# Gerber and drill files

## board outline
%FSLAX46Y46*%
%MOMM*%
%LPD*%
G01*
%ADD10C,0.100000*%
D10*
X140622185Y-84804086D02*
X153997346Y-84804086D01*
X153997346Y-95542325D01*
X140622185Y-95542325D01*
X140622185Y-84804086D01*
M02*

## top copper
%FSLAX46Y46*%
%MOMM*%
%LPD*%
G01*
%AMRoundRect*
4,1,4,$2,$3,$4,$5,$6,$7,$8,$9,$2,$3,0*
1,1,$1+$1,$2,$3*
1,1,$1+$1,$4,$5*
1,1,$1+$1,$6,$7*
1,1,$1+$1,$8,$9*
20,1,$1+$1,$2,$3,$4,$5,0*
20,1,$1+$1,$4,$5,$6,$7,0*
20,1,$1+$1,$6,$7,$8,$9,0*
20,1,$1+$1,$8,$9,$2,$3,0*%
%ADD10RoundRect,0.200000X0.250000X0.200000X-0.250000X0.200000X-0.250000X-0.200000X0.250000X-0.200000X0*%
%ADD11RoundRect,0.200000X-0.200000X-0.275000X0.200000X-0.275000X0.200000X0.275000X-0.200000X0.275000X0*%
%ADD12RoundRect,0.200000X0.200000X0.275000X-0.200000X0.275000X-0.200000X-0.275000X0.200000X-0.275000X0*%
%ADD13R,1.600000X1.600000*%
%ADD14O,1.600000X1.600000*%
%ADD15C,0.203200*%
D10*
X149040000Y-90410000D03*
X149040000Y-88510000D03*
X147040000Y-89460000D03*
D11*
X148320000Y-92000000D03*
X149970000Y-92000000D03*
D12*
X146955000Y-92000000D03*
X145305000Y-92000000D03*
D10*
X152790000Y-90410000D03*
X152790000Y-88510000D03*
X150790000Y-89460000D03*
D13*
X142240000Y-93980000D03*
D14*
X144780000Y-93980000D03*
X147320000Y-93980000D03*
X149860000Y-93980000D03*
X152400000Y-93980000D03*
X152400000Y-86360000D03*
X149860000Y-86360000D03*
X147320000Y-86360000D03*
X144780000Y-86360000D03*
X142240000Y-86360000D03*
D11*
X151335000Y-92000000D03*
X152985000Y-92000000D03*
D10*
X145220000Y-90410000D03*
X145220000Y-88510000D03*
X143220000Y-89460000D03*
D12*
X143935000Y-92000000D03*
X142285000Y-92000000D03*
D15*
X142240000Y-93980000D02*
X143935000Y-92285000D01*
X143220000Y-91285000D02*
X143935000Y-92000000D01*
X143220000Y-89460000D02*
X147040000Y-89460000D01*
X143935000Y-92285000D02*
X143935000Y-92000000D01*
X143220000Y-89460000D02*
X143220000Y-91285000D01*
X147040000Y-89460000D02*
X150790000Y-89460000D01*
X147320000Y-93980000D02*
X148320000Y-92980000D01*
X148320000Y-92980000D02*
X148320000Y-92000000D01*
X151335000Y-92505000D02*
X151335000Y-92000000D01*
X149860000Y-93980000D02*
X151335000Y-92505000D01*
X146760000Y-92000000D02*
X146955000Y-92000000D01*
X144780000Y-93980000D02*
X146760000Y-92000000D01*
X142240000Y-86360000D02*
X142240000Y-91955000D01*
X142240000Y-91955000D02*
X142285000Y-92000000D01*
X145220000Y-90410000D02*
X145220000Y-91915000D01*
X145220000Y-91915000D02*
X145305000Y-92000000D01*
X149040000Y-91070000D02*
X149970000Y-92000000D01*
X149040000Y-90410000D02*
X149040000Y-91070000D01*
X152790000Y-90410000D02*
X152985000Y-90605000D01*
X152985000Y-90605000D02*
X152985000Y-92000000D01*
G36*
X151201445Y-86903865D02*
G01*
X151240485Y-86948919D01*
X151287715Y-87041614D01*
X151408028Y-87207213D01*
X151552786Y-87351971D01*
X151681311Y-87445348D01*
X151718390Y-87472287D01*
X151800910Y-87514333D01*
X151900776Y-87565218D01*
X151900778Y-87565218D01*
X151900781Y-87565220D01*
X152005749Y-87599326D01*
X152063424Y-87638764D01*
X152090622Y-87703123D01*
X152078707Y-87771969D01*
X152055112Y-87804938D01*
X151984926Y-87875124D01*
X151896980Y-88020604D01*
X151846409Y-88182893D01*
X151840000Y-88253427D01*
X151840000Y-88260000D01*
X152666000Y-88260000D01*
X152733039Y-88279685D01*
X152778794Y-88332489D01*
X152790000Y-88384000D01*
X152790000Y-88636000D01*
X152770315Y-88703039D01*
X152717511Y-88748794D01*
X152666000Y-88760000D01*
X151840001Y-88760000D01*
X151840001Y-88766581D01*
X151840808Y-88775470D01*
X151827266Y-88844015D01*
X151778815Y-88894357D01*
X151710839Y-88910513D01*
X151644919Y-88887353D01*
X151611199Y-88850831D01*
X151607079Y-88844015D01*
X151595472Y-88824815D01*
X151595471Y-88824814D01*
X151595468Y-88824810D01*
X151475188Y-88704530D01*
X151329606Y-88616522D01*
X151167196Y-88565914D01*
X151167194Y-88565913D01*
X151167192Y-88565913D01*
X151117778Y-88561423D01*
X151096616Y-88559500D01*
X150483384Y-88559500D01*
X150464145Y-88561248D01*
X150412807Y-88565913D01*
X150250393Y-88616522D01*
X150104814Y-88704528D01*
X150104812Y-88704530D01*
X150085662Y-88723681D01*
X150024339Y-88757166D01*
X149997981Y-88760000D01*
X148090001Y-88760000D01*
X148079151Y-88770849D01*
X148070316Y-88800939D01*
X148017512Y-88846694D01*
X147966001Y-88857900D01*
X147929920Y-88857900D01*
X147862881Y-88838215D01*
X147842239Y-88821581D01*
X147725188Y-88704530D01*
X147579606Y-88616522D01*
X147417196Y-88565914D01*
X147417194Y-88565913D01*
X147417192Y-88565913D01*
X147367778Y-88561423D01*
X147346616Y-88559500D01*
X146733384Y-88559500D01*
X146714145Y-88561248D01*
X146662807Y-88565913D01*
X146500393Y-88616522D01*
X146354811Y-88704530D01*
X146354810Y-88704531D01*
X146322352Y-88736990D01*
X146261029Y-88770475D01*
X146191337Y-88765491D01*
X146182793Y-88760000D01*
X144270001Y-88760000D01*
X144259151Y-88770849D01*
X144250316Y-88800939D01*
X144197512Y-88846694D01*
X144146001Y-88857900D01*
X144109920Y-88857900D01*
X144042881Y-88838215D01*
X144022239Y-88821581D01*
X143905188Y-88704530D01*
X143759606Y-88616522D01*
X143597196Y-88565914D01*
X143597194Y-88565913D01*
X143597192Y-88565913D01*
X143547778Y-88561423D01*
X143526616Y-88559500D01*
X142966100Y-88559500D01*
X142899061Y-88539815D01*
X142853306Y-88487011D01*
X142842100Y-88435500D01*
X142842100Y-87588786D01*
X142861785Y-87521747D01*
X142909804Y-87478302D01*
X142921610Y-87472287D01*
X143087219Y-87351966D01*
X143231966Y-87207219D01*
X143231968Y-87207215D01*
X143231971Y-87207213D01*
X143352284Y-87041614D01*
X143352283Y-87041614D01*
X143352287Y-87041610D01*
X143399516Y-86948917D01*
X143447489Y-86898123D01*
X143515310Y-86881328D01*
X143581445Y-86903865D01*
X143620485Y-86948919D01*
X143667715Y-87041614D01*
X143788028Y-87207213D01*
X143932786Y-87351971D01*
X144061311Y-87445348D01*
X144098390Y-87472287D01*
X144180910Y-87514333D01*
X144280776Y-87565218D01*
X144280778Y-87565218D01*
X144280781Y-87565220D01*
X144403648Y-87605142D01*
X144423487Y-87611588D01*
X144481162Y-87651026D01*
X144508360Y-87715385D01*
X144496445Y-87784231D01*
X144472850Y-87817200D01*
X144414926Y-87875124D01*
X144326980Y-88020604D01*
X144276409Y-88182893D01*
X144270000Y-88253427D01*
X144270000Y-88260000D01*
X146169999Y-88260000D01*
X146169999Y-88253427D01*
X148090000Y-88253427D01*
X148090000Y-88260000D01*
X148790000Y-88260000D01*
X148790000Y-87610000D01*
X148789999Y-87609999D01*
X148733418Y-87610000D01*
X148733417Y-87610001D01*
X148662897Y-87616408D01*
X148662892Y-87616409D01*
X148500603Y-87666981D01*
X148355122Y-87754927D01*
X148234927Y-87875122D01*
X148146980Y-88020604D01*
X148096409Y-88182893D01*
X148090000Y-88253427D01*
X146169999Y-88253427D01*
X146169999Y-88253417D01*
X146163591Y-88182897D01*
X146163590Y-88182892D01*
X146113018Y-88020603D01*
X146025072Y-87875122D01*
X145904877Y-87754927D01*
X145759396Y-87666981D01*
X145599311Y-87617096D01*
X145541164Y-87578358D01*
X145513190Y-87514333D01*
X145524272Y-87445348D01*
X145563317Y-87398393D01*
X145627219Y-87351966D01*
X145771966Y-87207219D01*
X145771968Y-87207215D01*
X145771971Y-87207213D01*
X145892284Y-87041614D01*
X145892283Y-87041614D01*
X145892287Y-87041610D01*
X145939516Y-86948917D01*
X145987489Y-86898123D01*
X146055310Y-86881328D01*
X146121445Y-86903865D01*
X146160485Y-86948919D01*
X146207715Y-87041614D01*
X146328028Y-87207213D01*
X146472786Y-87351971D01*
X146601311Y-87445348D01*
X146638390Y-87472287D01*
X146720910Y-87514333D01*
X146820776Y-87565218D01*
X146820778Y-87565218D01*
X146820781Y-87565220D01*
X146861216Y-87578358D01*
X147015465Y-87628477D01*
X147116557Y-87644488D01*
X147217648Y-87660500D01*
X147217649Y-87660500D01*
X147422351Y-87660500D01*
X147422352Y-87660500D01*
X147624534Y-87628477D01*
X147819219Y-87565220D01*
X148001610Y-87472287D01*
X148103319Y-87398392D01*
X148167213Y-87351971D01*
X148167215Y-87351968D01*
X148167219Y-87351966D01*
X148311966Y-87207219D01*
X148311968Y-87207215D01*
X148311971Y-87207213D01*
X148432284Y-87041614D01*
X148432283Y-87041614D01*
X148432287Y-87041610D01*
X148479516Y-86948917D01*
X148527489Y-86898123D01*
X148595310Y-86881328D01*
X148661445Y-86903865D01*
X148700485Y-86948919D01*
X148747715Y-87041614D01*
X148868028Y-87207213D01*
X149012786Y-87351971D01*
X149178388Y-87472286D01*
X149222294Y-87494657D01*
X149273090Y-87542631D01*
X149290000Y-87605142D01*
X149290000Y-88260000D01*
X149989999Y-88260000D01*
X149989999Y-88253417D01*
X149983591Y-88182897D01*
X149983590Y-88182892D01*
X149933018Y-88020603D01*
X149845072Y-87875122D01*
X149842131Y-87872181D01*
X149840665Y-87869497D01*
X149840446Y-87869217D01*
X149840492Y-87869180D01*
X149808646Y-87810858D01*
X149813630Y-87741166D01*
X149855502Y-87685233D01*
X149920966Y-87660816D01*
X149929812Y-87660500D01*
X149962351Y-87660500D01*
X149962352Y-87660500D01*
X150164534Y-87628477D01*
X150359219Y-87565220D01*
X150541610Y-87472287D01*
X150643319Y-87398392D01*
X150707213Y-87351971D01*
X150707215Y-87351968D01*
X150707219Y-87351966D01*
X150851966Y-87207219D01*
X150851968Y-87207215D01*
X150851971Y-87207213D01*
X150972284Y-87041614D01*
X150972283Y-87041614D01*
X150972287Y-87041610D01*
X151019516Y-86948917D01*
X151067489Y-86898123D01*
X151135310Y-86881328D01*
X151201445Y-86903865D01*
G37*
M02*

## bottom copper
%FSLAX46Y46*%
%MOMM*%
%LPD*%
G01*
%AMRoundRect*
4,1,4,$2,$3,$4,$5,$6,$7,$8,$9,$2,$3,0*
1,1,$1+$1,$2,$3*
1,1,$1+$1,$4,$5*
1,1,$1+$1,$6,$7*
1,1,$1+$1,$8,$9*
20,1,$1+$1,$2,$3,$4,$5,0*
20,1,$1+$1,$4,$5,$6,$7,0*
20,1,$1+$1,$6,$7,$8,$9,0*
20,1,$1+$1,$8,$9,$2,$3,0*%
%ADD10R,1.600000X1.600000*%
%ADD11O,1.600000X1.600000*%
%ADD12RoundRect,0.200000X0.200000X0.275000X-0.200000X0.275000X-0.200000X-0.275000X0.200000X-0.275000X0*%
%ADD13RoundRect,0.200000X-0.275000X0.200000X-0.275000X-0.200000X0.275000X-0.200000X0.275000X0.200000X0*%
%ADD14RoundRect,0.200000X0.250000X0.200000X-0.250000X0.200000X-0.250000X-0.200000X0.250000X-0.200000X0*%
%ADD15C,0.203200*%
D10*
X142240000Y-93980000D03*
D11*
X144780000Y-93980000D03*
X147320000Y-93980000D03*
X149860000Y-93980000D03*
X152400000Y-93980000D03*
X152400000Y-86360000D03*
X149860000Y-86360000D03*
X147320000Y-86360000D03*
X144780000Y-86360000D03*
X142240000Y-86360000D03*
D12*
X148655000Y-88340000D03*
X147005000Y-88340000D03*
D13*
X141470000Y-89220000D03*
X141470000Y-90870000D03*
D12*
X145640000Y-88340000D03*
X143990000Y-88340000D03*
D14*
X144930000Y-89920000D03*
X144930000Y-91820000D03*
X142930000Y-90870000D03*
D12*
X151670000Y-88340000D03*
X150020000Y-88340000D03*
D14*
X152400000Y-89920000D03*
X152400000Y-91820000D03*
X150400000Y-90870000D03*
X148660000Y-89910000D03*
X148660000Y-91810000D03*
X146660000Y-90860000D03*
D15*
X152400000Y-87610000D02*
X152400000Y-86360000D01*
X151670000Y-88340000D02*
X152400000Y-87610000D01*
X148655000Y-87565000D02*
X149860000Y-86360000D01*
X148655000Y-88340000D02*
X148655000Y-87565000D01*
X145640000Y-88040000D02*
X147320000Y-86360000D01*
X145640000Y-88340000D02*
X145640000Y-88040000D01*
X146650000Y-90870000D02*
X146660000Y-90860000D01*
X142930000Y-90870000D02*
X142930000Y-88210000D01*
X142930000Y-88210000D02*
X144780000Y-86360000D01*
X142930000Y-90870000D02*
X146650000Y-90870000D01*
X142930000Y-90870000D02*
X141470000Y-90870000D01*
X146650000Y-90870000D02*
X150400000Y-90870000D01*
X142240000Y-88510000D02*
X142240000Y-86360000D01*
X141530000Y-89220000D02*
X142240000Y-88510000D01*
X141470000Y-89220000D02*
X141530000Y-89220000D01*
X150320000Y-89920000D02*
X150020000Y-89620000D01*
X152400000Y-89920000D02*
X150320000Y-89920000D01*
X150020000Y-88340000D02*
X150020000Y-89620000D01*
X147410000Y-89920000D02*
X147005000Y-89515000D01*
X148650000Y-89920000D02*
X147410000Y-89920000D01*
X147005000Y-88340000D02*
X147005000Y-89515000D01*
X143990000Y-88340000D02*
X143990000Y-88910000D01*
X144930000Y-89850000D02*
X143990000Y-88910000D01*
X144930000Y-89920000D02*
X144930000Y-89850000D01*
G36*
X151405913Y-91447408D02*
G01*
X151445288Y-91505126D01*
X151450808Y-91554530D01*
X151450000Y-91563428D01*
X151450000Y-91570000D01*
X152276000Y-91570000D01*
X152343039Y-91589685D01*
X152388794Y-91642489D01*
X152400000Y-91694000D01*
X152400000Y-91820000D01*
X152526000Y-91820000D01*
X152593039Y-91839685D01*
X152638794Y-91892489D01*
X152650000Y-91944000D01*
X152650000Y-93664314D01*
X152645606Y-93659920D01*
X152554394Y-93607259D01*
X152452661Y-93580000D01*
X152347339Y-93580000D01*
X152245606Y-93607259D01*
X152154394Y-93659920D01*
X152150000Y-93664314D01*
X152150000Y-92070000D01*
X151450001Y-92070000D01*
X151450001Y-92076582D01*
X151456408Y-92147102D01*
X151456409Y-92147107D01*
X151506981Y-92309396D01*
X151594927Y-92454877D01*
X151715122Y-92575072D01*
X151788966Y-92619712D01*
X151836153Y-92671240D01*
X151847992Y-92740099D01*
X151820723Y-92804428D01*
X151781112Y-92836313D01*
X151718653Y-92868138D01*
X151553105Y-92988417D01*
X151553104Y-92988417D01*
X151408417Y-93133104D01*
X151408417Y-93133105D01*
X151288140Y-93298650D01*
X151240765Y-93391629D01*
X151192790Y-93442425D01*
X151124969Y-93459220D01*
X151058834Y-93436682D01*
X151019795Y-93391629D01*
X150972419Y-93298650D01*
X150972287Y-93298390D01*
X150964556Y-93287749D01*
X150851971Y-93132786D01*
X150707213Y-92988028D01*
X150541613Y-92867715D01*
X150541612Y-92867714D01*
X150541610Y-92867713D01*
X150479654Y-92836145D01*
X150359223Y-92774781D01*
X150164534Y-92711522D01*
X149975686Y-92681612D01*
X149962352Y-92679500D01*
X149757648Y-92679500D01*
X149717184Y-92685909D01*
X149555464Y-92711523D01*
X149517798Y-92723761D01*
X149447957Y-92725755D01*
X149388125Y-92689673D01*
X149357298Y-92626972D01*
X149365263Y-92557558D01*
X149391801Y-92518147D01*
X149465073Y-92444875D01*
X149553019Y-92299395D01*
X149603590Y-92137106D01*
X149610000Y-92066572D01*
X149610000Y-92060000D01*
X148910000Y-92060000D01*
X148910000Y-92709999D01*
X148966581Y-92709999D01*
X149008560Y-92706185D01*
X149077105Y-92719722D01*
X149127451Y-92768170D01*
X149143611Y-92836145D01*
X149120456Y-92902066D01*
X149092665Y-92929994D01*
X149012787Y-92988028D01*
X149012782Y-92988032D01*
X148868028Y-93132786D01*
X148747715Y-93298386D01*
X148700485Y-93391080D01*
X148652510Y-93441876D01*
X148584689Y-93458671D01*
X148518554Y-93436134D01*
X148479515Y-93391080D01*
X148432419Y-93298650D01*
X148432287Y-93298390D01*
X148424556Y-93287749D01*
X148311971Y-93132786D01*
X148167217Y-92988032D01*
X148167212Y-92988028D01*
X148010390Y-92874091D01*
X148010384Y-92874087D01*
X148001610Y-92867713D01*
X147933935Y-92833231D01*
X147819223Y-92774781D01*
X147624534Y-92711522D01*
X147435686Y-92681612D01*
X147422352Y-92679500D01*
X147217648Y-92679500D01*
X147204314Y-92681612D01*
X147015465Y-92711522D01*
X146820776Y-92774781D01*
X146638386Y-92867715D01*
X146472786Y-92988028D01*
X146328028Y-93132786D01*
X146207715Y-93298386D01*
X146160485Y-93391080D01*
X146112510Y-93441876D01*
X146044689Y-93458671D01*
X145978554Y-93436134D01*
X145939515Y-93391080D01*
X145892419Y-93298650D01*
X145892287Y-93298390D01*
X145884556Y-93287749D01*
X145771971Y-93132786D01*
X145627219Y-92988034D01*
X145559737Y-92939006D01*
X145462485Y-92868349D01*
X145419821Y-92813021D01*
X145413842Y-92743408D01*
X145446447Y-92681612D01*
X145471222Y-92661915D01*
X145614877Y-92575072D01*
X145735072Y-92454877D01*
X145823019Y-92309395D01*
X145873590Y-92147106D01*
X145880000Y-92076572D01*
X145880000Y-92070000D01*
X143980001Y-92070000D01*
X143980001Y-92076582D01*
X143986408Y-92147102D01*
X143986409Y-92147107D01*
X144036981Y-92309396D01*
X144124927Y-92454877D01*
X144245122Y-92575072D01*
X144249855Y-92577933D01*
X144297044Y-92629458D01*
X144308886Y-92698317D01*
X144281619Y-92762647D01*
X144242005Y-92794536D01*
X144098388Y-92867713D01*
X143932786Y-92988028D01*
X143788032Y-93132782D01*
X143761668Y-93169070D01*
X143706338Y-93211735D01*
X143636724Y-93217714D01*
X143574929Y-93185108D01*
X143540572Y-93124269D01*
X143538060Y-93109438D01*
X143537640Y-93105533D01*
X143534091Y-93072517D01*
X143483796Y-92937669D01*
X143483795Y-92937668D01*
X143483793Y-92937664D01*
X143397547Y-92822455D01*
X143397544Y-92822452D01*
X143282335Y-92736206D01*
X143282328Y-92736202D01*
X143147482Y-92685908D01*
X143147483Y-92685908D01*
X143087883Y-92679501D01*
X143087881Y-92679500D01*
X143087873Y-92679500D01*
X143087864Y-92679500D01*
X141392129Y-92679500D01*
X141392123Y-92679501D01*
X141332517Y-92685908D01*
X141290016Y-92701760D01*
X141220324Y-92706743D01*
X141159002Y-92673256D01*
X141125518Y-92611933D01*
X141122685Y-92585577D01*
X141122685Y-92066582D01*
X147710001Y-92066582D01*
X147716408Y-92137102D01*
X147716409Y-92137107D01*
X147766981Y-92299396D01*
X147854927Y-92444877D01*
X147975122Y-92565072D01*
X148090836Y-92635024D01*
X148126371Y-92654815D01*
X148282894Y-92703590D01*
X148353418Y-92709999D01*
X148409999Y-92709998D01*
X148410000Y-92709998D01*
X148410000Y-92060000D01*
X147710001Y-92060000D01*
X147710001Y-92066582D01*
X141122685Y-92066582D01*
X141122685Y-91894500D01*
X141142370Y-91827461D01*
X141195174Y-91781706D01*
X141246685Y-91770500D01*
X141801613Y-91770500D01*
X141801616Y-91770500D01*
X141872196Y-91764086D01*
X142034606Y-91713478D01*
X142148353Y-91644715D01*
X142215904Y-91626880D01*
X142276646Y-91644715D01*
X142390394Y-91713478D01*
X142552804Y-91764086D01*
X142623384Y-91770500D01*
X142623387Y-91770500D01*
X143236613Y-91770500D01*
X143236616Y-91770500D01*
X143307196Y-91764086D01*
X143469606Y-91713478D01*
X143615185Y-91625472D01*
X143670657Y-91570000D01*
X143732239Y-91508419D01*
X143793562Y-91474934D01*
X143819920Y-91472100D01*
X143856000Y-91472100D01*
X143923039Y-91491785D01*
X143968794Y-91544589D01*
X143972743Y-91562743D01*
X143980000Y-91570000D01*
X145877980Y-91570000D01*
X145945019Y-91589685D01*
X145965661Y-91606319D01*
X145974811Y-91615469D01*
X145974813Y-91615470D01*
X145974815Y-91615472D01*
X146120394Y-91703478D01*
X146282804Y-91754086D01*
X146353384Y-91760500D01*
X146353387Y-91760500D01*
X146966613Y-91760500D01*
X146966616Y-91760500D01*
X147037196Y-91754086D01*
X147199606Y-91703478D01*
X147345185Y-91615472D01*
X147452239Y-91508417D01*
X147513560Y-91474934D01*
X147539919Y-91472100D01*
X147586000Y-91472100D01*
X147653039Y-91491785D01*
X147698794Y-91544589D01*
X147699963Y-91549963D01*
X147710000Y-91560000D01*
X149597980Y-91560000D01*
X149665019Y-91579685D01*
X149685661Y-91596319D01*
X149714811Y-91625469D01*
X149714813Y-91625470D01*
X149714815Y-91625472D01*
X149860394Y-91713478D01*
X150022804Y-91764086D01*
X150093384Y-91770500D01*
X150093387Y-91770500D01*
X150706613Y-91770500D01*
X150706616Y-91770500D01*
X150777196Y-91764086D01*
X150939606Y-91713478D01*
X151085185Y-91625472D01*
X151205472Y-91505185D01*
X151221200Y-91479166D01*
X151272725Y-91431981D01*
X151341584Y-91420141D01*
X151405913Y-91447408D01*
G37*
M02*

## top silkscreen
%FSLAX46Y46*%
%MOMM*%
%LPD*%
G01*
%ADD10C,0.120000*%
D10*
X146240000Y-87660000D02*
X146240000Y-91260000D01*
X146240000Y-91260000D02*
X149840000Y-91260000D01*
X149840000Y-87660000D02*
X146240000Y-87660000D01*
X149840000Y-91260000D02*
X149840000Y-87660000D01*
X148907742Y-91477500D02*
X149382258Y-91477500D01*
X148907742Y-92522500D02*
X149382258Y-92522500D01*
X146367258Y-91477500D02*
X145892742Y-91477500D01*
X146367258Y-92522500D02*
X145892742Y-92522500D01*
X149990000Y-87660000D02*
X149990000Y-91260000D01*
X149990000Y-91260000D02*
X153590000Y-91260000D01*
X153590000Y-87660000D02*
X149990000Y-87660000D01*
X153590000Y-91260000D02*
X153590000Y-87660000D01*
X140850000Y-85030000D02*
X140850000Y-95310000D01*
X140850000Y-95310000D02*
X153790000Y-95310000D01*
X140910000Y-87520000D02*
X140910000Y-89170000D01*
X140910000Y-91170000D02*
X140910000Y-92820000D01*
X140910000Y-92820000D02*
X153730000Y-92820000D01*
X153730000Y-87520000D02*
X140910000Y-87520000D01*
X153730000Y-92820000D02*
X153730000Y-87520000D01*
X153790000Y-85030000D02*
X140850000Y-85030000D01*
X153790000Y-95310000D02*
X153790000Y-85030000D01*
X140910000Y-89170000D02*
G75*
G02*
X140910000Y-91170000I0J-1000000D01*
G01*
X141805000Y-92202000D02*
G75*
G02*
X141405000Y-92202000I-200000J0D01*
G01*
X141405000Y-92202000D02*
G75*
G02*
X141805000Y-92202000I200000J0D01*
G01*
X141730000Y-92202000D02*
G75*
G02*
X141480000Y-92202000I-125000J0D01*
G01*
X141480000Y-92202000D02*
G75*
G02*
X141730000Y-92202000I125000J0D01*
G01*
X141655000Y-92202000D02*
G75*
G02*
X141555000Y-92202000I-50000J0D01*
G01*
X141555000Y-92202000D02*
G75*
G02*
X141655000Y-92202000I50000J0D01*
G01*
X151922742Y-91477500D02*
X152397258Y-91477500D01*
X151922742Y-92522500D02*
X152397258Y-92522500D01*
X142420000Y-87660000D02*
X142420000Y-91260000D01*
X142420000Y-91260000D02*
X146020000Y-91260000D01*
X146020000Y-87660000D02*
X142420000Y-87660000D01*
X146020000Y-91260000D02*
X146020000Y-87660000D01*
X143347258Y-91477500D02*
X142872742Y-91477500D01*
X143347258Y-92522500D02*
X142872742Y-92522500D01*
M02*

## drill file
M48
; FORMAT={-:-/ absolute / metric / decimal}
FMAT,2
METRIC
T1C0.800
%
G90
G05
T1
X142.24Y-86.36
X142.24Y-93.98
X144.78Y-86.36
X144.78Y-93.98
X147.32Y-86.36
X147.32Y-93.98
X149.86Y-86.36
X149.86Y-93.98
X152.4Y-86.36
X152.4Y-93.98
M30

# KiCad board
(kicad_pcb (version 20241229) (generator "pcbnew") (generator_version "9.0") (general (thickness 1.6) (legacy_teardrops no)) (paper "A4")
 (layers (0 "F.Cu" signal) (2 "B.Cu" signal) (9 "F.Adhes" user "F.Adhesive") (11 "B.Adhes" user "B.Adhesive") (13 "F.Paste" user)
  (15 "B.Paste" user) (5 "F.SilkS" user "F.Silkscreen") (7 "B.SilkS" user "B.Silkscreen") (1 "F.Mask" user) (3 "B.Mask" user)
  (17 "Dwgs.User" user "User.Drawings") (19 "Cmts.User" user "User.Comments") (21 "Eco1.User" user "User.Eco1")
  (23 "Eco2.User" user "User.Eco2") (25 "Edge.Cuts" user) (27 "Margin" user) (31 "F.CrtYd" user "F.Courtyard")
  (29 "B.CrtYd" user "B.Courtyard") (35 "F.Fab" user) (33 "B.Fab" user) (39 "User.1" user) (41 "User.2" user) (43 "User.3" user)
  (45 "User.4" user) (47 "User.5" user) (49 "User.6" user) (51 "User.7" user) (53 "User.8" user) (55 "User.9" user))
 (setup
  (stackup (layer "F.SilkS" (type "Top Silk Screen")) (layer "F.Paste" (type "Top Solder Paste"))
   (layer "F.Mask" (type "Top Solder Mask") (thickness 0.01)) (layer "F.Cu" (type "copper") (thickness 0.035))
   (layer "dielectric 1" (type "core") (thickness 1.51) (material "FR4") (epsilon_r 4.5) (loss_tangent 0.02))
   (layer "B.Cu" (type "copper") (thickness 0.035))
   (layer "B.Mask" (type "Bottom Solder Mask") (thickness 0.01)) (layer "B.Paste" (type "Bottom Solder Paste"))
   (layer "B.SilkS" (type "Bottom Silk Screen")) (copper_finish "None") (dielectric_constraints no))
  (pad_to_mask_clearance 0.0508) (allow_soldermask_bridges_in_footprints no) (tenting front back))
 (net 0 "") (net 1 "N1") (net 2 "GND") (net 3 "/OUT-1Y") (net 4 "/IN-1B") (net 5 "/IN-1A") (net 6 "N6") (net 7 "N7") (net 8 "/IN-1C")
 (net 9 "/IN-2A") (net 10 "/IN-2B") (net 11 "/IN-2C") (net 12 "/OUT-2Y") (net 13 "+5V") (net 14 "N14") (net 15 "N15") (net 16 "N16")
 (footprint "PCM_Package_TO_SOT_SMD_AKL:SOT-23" (layer "F.Cu") (at 148.04 89.46 180)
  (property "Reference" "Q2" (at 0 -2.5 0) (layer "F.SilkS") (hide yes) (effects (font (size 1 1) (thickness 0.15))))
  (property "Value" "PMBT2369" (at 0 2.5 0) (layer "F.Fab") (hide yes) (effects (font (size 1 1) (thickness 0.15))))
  (fp_line (start 1.8 1.8) (end 1.8 -1.8) (stroke (width 0.12) (type solid)) (layer "F.SilkS"))
  (fp_line (start 1.8 -1.8) (end -1.8 -1.8) (stroke (width 0.12) (type solid)) (layer "F.SilkS"))
  (fp_line (start -1.8 1.8) (end 1.8 1.8) (stroke (width 0.12) (type solid)) (layer "F.SilkS"))
  (fp_line (start -1.8 -1.8) (end -1.8 1.8) (stroke (width 0.12) (type solid)) (layer "F.SilkS"))
  (pad "1" smd roundrect (at -1 -0.95 180) (size 0.9 0.8) (layers "F.Cu" "F.Mask" "F.Paste") (roundrect_rratio 0.25) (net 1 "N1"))
  (pad "2" smd roundrect (at -1 0.95 180) (size 0.9 0.8) (layers "F.Cu" "F.Mask" "F.Paste") (roundrect_rratio 0.25) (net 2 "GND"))
  (pad "3" smd roundrect (at 1 0 180) (size 0.9 0.8) (layers "F.Cu" "F.Mask" "F.Paste") (roundrect_rratio 0.25) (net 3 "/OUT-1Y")))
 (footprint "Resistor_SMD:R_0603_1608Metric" (layer "F.Cu") (at 149.145 92)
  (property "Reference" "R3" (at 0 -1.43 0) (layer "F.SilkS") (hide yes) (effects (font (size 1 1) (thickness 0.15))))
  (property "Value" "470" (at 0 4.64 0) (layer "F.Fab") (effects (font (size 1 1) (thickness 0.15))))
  (fp_line (start -0.237258 -0.5225) (end 0.237258 -0.5225) (stroke (width 0.12) (type solid)) (layer "F.SilkS"))
  (fp_line (start -0.237258 0.5225) (end 0.237258 0.5225) (stroke (width 0.12) (type solid)) (layer "F.SilkS"))
  (pad "1" smd roundrect (at -0.825 0) (size 0.8 0.95) (layers "F.Cu" "F.Mask" "F.Paste") (roundrect_rratio 0.25) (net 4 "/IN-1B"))
  (pad "2" smd roundrect (at 0.825 0) (size 0.8 0.95) (layers "F.Cu" "F.Mask" "F.Paste") (roundrect_rratio 0.25) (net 1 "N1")))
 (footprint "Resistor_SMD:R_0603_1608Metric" (layer "F.Cu") (at 146.13 92 180)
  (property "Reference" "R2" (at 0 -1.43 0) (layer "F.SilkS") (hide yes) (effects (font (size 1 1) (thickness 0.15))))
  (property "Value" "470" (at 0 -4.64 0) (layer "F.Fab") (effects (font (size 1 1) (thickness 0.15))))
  (fp_line (start -0.237258 0.5225) (end 0.237258 0.5225) (stroke (width 0.12) (type solid)) (layer "F.SilkS"))
  (fp_line (start -0.237258 -0.5225) (end 0.237258 -0.5225) (stroke (width 0.12) (type solid)) (layer "F.SilkS"))
  (pad "1" smd roundrect (at -0.825 0 180) (size 0.8 0.95) (layers "F.Cu" "F.Mask" "F.Paste") (roundrect_rratio 0.25) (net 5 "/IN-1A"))
  (pad "2" smd roundrect (at 0.825 0 180) (size 0.8 0.95) (layers "F.Cu" "F.Mask" "F.Paste") (roundrect_rratio 0.25) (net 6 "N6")))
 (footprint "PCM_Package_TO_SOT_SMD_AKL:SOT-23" (layer "F.Cu") (at 151.79 89.46 180)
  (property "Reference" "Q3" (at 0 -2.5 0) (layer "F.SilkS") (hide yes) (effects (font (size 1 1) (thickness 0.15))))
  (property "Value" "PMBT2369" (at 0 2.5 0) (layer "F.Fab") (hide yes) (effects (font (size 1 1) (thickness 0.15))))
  (fp_line (start 1.8 1.8) (end 1.8 -1.8) (stroke (width 0.12) (type solid)) (layer "F.SilkS"))
  (fp_line (start 1.8 -1.8) (end -1.8 -1.8) (stroke (width 0.12) (type solid)) (layer "F.SilkS"))
  (fp_line (start -1.8 1.8) (end 1.8 1.8) (stroke (width 0.12) (type solid)) (layer "F.SilkS"))
  (fp_line (start -1.8 -1.8) (end -1.8 1.8) (stroke (width 0.12) (type solid)) (layer "F.SilkS"))
  (pad "1" smd roundrect (at -1 -0.95 180) (size 0.9 0.8) (layers "F.Cu" "F.Mask" "F.Paste") (roundrect_rratio 0.25) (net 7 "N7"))
  (pad "2" smd roundrect (at -1 0.95 180) (size 0.9 0.8) (layers "F.Cu" "F.Mask" "F.Paste") (roundrect_rratio 0.25) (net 2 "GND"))
  (pad "3" smd roundrect (at 1 0 180) (size 0.9 0.8) (layers "F.Cu" "F.Mask" "F.Paste") (roundrect_rratio 0.25) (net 3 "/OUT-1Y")))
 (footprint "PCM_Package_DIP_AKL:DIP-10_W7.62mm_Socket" (layer "F.Cu") (at 142.24 93.98 90)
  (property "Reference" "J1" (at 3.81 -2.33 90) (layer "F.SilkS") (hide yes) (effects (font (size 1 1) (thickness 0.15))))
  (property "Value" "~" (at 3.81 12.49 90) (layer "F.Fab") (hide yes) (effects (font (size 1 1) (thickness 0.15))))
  (fp_line (start 8.95 -1.39) (end -1.33 -1.39) (stroke (width 0.12) (type solid)) (layer "F.SilkS"))
  (fp_line (start -1.33 -1.39) (end -1.33 11.55) (stroke (width 0.12) (type solid)) (layer "F.SilkS"))
  (fp_line (start 6.46 -1.33) (end 4.81 -1.33) (stroke (width 0.12) (type solid)) (layer "F.SilkS"))
  (fp_line (start 2.81 -1.33) (end 1.16 -1.33) (stroke (width 0.12) (type solid)) (layer "F.SilkS"))
  (fp_line (start 1.16 -1.33) (end 1.16 11.49) (stroke (width 0.12) (type solid)) (layer "F.SilkS"))
  (fp_line (start 6.46 11.49) (end 6.46 -1.33) (stroke (width 0.12) (type solid)) (layer "F.SilkS"))
  (fp_line (start 1.16 11.49) (end 6.46 11.49) (stroke (width 0.12) (type solid)) (layer "F.SilkS"))
  (fp_line (start 8.95 11.55) (end 8.95 -1.39) (stroke (width 0.12) (type solid)) (layer "F.SilkS"))
  (fp_line (start -1.33 11.55) (end 8.95 11.55) (stroke (width 0.12) (type solid)) (layer "F.SilkS"))
  (fp_arc (start 4.81 -1.33) (mid 3.81 -0.33) (end 2.81 -1.33) (stroke (width 0.12) (type solid)) (layer "F.SilkS"))
  (fp_circle (center 1.778 -0.635) (end 1.978 -0.635) (stroke (width 0.12) (type solid)) (fill no) (layer "F.SilkS"))
  (fp_circle (center 1.778 -0.635) (end 1.903 -0.635) (stroke (width 0.12) (type solid)) (fill no) (layer "F.SilkS"))
  (fp_circle (center 1.778 -0.635) (end 1.828 -0.635) (stroke (width 0.12) (type solid)) (fill no) (layer "F.SilkS"))
  (pad "1" thru_hole rect (at 0 0 90) (size 1.6 1.6) (drill 0.8) (layers "*.Cu" "*.Mask") (remove_unused_layers no) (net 3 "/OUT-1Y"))
  (pad "2" thru_hole oval (at 0 2.54 90) (size 1.6 1.6) (drill 0.8) (layers "*.Cu" "*.Mask") (remove_unused_layers no) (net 5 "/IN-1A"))
  (pad "3" thru_hole oval (at 0 5.08 90) (size 1.6 1.6) (drill 0.8) (layers "*.Cu" "*.Mask") (remove_unused_layers no) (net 4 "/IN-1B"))
  (pad "4" thru_hole oval (at 0 7.62 90) (size 1.6 1.6) (drill 0.8) (layers "*.Cu" "*.Mask") (remove_unused_layers no) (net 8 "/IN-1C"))
  (pad "5" thru_hole oval (at 0 10.16 90) (size 1.6 1.6) (drill 0.8) (layers "*.Cu" "*.Mask") (remove_unused_layers no) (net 2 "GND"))
  (pad "6" thru_hole oval (at 7.62 10.16 90) (size 1.6 1.6) (drill 0.8) (layers "*.Cu" "*.Mask") (remove_unused_layers no) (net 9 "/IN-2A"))
  (pad "7" thru_hole oval (at 7.62 7.62 90) (size 1.6 1.6) (drill 0.8) (layers "*.Cu" "*.Mask") (remove_unused_layers no) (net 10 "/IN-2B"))
  (pad "8" thru_hole oval (at 7.62 5.08 90) (size 1.6 1.6) (drill 0.8) (layers "*.Cu" "*.Mask") (remove_unused_layers no) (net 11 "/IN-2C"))
  (pad "9" thru_hole oval (at 7.62 2.54 90) (size 1.6 1.6) (drill 0.8) (layers "*.Cu" "*.Mask") (remove_unused_layers no) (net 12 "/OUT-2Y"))
  (pad "10" thru_hole oval (at 7.62 0 90) (size 1.6 1.6) (drill 0.8) (layers "*.Cu" "*.Mask") (remove_unused_layers no) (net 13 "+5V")))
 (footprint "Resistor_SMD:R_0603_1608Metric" (layer "F.Cu") (at 152.16 92)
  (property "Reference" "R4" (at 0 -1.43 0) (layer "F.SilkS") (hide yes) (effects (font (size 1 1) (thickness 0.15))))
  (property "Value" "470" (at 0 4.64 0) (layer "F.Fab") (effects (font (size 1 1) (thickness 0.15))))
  (fp_line (start -0.237258 -0.5225) (end 0.237258 -0.5225) (stroke (width 0.12) (type solid)) (layer "F.SilkS"))
  (fp_line (start -0.237258 0.5225) (end 0.237258 0.5225) (stroke (width 0.12) (type solid)) (layer "F.SilkS"))
  (pad "1" smd roundrect (at -0.825 0) (size 0.8 0.95) (layers "F.Cu" "F.Mask" "F.Paste") (roundrect_rratio 0.25) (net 8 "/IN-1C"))
  (pad "2" smd roundrect (at 0.825 0) (size 0.8 0.95) (layers "F.Cu" "F.Mask" "F.Paste") (roundrect_rratio 0.25) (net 7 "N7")))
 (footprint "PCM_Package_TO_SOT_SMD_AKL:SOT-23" (layer "F.Cu") (at 144.22 89.46 180)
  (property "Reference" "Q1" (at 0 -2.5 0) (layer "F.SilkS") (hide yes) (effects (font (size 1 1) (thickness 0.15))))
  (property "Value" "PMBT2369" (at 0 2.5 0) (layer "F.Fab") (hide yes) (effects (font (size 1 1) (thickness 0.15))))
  (fp_line (start 1.8 1.8) (end 1.8 -1.8) (stroke (width 0.12) (type solid)) (layer "F.SilkS"))
  (fp_line (start 1.8 -1.8) (end -1.8 -1.8) (stroke (width 0.12) (type solid)) (layer "F.SilkS"))
  (fp_line (start -1.8 1.8) (end 1.8 1.8) (stroke (width 0.12) (type solid)) (layer "F.SilkS"))
  (fp_line (start -1.8 -1.8) (end -1.8 1.8) (stroke (width 0.12) (type solid)) (layer "F.SilkS"))
  (pad "1" smd roundrect (at -1 -0.95 180) (size 0.9 0.8) (layers "F.Cu" "F.Mask" "F.Paste") (roundrect_rratio 0.25) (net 6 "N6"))
  (pad "2" smd roundrect (at -1 0.95 180) (size 0.9 0.8) (layers "F.Cu" "F.Mask" "F.Paste") (roundrect_rratio 0.25) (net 2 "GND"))
  (pad "3" smd roundrect (at 1 0 180) (size 0.9 0.8) (layers "F.Cu" "F.Mask" "F.Paste") (roundrect_rratio 0.25) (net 3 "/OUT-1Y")))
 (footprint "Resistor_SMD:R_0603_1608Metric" (layer "F.Cu") (at 143.11 92 180)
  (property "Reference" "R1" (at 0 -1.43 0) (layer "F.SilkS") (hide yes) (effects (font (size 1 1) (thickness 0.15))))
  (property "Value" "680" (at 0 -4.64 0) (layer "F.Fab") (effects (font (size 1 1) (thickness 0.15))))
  (fp_line (start -0.237258 0.5225) (end 0.237258 0.5225) (stroke (width 0.12) (type solid)) (layer "F.SilkS"))
  (fp_line (start -0.237258 -0.5225) (end 0.237258 -0.5225) (stroke (width 0.12) (type solid)) (layer "F.SilkS"))
  (pad "1" smd roundrect (at -0.825 0 180) (size 0.8 0.95) (layers "F.Cu" "F.Mask" "F.Paste") (roundrect_rratio 0.25) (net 3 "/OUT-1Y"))
  (pad "2" smd roundrect (at 0.825 0 180) (size 0.8 0.95) (layers "F.Cu" "F.Mask" "F.Paste") (roundrect_rratio 0.25) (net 13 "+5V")))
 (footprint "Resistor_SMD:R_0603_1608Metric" (layer "B.Cu") (at 147.83 88.34 180)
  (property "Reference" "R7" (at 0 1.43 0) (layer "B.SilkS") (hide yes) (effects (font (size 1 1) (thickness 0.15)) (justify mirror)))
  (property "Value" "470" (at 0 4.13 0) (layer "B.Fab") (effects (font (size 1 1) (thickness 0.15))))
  (pad "1" smd roundrect (at -0.825 0 180) (size 0.8 0.95) (layers "B.Cu" "B.Mask" "B.Paste") (roundrect_rratio 0.25) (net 10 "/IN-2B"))
  (pad "2" smd roundrect (at 0.825 0 180) (size 0.8 0.95) (layers "B.Cu" "B.Mask" "B.Paste") (roundrect_rratio 0.25) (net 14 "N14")))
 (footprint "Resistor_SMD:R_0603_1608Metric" (layer "B.Cu") (at 141.47 90.045 -90)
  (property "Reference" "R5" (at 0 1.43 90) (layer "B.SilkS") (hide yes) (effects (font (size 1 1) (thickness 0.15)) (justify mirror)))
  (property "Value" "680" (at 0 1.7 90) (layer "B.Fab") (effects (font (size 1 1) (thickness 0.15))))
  (pad "1" smd roundrect (at -0.825 0 270) (size 0.8 0.95) (layers "B.Cu" "B.Mask" "B.Paste") (roundrect_rratio 0.25) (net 13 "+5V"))
  (pad "2" smd roundrect (at 0.825 0 270) (size 0.8 0.95) (layers "B.Cu" "B.Mask" "B.Paste") (roundrect_rratio 0.25) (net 12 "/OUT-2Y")))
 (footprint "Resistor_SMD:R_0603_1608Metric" (layer "B.Cu") (at 144.815 88.34 180)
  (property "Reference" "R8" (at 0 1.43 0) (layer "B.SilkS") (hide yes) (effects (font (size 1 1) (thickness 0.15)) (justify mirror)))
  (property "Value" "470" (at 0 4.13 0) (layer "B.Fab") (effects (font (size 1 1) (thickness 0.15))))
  (pad "1" smd roundrect (at -0.825 0 180) (size 0.8 0.95) (layers "B.Cu" "B.Mask" "B.Paste") (roundrect_rratio 0.25) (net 11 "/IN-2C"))
  (pad "2" smd roundrect (at 0.825 0 180) (size 0.8 0.95) (layers "B.Cu" "B.Mask" "B.Paste") (roundrect_rratio 0.25) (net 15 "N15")))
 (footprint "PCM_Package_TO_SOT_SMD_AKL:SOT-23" (layer "B.Cu") (at 143.93 90.87 180)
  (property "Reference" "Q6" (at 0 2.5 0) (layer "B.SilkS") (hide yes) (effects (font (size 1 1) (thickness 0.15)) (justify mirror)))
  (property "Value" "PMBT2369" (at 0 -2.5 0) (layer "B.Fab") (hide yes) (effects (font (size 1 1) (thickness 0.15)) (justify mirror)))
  (pad "1" smd roundrect (at -1 0.95 180) (size 0.9 0.8) (layers "B.Cu" "B.Mask" "B.Paste") (roundrect_rratio 0.25) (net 15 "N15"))
  (pad "2" smd roundrect (at -1 -0.95 180) (size 0.9 0.8) (layers "B.Cu" "B.Mask" "B.Paste") (roundrect_rratio 0.25) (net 2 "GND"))
  (pad "3" smd roundrect (at 1 0 180) (size 0.9 0.8) (layers "B.Cu" "B.Mask" "B.Paste") (roundrect_rratio 0.25) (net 12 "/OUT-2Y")))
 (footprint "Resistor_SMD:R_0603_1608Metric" (layer "B.Cu") (at 150.845 88.34 180)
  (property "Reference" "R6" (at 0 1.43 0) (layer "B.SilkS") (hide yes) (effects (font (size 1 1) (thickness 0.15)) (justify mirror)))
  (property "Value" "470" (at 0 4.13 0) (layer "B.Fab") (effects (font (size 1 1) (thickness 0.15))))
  (pad "1" smd roundrect (at -0.825 0 180) (size 0.8 0.95) (layers "B.Cu" "B.Mask" "B.Paste") (roundrect_rratio 0.25) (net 9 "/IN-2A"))
  (pad "2" smd roundrect (at 0.825 0 180) (size 0.8 0.95) (layers "B.Cu" "B.Mask" "B.Paste") (roundrect_rratio 0.25) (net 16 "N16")))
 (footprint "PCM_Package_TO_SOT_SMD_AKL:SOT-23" (layer "B.Cu") (at 151.4 90.87 180)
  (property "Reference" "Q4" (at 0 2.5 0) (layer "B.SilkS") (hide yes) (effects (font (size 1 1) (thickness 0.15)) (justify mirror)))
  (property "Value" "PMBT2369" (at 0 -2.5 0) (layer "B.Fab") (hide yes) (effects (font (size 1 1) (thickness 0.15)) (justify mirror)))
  (pad "1" smd roundrect (at -1 0.95 180) (size 0.9 0.8) (layers "B.Cu" "B.Mask" "B.Paste") (roundrect_rratio 0.25) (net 16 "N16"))
  (pad "2" smd roundrect (at -1 -0.95 180) (size 0.9 0.8) (layers "B.Cu" "B.Mask" "B.Paste") (roundrect_rratio 0.25) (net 2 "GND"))
  (pad "3" smd roundrect (at 1 0 180) (size 0.9 0.8) (layers "B.Cu" "B.Mask" "B.Paste") (roundrect_rratio 0.25) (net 12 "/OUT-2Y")))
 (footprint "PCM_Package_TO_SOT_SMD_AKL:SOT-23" (layer "B.Cu") (at 147.66 90.86 180)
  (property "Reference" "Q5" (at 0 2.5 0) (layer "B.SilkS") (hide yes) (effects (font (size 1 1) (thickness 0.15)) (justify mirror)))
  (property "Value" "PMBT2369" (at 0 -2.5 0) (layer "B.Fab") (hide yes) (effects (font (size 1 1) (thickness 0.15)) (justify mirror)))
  (pad "1" smd roundrect (at -1 0.95 180) (size 0.9 0.8) (layers "B.Cu" "B.Mask" "B.Paste") (roundrect_rratio 0.25) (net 14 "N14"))
  (pad "2" smd roundrect (at -1 -0.95 180) (size 0.9 0.8) (layers "B.Cu" "B.Mask" "B.Paste") (roundrect_rratio 0.25) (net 2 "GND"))
  (pad "3" smd roundrect (at 1 0 180) (size 0.9 0.8) (layers "B.Cu" "B.Mask" "B.Paste") (roundrect_rratio 0.25) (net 12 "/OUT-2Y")))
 (gr_rect (start 140.622185 84.804086) (end 153.997346 95.542325) (stroke (width 0.1) (type default)) (fill no) (layer "Edge.Cuts"))
 (segment (start 142.24 93.98) (end 143.935 92.285) (width 0.2032) (layer "F.Cu") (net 3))
 (segment (start 143.22 91.285) (end 143.935 92) (width 0.2032) (layer "F.Cu") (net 3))
 (segment (start 143.22 89.46) (end 147.04 89.46) (width 0.2032) (layer "F.Cu") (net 3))
 (segment (start 143.935 92.285) (end 143.935 92) (width 0.2032) (layer "F.Cu") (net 3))
 (segment (start 143.22 89.46) (end 143.22 91.285) (width 0.2032) (layer "F.Cu") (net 3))
 (segment (start 147.04 89.46) (end 150.79 89.46) (width 0.2032) (layer "F.Cu") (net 3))
 (segment (start 147.32 93.98) (end 148.32 92.98) (width 0.2032) (layer "F.Cu") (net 4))
 (segment (start 148.32 92.98) (end 148.32 92) (width 0.2032) (layer "F.Cu") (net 4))
 (segment (start 151.335 92.505) (end 151.335 92) (width 0.2032) (layer "F.Cu") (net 8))
 (segment (start 149.86 93.98) (end 151.335 92.505) (width 0.2032) (layer "F.Cu") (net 8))
 (segment (start 146.76 92) (end 146.955 92) (width 0.2032) (layer "F.Cu") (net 5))
 (segment (start 144.78 93.98) (end 146.76 92) (width 0.2032) (layer "F.Cu") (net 5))
 (segment (start 152.4 87.61) (end 152.4 86.36) (width 0.2032) (layer "B.Cu") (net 9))
 (segment (start 151.67 88.34) (end 152.4 87.61) (width 0.2032) (layer "B.Cu") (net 9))
 (segment (start 148.655 87.565) (end 149.86 86.36) (width 0.2032) (layer "B.Cu") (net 10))
 (segment (start 148.655 88.34) (end 148.655 87.565) (width 0.2032) (layer "B.Cu") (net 10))
 (segment (start 145.64 88.04) (end 147.32 86.36) (width 0.2032) (layer "B.Cu") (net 11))
 (segment (start 145.64 88.34) (end 145.64 88.04) (width 0.2032) (layer "B.Cu") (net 11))
 (segment (start 146.65 90.87) (end 146.66 90.86) (width 0.2032) (layer "B.Cu") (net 12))
 (segment (start 142.93 90.87) (end 142.93 88.21) (width 0.2032) (layer "B.Cu") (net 12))
 (segment (start 142.93 88.21) (end 144.78 86.36) (width 0.2032) (layer "B.Cu") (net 12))
 (segment (start 142.93 90.87) (end 146.65 90.87) (width 0.2032) (layer "B.Cu") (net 12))
 (segment (start 142.93 90.87) (end 141.47 90.87) (width 0.2032) (layer "B.Cu") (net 12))
 (segment (start 146.65 90.87) (end 150.4 90.87) (width 0.2032) (layer "B.Cu") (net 12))
 (segment (start 142.24 86.36) (end 142.24 91.955) (width 0.2032) (layer "F.Cu") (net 13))
 (segment (start 142.24 91.955) (end 142.285 92) (width 0.2032) (layer "F.Cu") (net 13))
 (segment (start 142.24 88.51) (end 142.24 86.36) (width 0.2032) (layer "B.Cu") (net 13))
 (segment (start 141.53 89.22) (end 142.24 88.51) (width 0.2032) (layer "B.Cu") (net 13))
 (segment (start 141.47 89.22) (end 141.53 89.22) (width 0.2032) (layer "B.Cu") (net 13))
 (segment (start 145.22 90.41) (end 145.22 91.915) (width 0.2032) (layer "F.Cu") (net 6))
 (segment (start 145.22 91.915) (end 145.305 92) (width 0.2032) (layer "F.Cu") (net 6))
 (segment (start 149.04 91.07) (end 149.97 92) (width 0.2032) (layer "F.Cu") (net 1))
 (segment (start 149.04 90.41) (end 149.04 91.07) (width 0.2032) (layer "F.Cu") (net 1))
 (segment (start 152.79 90.41) (end 152.985 90.605) (width 0.2032) (layer "F.Cu") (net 7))
 (segment (start 152.985 90.605) (end 152.985 92) (width 0.2032) (layer "F.Cu") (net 7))
 (segment (start 150.32 89.92) (end 150.02 89.62) (width 0.2032) (layer "B.Cu") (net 16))
 (segment (start 152.4 89.92) (end 150.32 89.92) (width 0.2032) (layer "B.Cu") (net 16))
 (segment (start 150.02 88.34) (end 150.02 89.62) (width 0.2032) (layer "B.Cu") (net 16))
 (segment (start 147.41 89.92) (end 147.005 89.515) (width 0.2032) (layer "B.Cu") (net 14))
 (segment (start 148.65 89.92) (end 147.41 89.92) (width 0.2032) (layer "B.Cu") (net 14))
 (segment (start 147.005 88.34) (end 147.005 89.515) (width 0.2032) (layer "B.Cu") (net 14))
 (segment (start 143.99 88.34) (end 143.99 88.91) (width 0.2032) (layer "B.Cu") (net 15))
 (segment (start 144.93 89.85) (end 143.99 88.91) (width 0.2032) (layer "B.Cu") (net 15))
 (segment (start 144.93 89.92) (end 144.93 89.85) (width 0.2032) (layer "B.Cu") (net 15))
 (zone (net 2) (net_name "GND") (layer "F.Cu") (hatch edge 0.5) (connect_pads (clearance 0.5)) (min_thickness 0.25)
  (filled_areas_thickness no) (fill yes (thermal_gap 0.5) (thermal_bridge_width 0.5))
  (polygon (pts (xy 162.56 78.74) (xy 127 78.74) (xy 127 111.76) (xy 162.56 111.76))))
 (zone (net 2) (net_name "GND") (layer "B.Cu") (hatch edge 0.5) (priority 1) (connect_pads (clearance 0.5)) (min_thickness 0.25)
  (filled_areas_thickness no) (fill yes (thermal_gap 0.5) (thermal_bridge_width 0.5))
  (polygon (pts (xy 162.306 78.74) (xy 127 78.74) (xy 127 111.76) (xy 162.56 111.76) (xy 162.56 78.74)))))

